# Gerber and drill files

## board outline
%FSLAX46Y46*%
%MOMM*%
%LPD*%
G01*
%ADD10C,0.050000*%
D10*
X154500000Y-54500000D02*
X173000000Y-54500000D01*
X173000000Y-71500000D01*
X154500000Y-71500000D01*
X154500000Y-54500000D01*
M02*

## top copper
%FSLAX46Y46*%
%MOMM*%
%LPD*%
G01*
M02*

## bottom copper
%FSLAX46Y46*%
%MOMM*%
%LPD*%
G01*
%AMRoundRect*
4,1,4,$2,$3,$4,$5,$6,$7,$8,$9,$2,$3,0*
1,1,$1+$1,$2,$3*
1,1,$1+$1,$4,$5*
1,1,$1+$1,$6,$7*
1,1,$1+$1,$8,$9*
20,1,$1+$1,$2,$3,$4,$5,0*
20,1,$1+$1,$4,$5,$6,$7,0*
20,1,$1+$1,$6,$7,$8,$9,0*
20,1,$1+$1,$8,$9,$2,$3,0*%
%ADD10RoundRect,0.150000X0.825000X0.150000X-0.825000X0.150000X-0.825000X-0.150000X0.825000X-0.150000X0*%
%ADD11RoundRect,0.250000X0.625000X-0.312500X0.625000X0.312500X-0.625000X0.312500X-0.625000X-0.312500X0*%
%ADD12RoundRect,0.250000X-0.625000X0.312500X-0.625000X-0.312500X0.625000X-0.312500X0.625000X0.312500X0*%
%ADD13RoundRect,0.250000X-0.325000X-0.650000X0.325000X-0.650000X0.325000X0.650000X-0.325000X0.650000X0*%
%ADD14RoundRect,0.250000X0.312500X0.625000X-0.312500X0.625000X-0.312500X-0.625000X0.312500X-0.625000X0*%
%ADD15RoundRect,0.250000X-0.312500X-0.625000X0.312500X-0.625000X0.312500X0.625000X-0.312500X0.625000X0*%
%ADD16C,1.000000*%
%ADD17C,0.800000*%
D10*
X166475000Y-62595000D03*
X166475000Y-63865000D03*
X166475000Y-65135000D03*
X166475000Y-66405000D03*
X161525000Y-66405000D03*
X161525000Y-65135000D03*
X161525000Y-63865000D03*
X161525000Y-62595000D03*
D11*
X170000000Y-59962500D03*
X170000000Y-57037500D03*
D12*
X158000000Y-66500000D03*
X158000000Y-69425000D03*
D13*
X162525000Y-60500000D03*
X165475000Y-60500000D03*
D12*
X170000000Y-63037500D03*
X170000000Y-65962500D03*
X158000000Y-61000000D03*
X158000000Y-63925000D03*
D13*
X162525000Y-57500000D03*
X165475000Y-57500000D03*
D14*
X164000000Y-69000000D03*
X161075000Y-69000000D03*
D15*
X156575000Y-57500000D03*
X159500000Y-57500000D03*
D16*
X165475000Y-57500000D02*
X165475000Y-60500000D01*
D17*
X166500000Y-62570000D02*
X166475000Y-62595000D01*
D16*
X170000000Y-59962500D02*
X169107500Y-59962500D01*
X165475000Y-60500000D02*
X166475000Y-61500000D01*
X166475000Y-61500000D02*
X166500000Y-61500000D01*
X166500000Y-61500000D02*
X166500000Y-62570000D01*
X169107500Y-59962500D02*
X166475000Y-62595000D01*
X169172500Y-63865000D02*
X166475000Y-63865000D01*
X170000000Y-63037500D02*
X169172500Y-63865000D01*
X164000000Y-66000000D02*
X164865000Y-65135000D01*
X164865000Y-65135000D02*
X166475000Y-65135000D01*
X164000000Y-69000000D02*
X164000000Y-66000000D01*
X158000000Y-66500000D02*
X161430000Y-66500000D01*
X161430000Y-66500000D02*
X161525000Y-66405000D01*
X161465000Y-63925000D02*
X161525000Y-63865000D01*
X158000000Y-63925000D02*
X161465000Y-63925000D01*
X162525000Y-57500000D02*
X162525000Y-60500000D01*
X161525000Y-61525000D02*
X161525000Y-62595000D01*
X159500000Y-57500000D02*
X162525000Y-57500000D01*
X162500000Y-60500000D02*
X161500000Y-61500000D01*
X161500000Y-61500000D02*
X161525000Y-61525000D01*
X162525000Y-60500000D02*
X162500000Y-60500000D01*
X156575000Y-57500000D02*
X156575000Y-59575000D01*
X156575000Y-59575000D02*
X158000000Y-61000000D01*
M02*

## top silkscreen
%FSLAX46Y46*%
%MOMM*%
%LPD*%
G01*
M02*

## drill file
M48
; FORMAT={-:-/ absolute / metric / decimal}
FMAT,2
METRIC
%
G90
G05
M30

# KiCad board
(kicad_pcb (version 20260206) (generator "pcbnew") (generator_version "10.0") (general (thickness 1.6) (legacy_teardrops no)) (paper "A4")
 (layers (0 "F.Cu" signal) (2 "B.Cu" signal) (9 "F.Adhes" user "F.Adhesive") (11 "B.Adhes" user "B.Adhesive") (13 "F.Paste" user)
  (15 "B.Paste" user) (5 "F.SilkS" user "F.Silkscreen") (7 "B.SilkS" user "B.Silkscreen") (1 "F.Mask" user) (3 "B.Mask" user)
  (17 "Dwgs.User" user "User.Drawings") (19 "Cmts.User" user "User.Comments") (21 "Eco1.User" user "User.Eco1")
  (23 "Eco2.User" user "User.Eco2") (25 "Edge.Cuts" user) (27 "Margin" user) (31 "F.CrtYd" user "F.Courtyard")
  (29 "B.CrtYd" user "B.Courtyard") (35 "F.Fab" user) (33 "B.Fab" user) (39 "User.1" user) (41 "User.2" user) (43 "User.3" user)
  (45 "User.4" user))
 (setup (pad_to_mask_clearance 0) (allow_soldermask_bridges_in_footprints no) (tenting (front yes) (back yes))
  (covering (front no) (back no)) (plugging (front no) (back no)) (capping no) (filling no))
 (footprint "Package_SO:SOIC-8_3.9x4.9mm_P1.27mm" (layer "B.Cu") (at 164 64.5 180)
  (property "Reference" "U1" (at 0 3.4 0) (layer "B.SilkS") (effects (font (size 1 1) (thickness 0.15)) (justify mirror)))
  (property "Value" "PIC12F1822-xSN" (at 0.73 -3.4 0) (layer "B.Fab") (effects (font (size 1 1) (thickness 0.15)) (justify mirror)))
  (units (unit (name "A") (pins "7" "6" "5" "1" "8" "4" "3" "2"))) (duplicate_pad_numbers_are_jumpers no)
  (pad "1" smd roundrect (at -2.475 1.905 180) (size 1.95 0.6) (layers "B.Cu" "B.Mask" "B.Paste") (roundrect_rratio 0.25)
   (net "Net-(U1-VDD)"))
  (pad "2" smd roundrect (at -2.475 0.635 180) (size 1.95 0.6) (layers "B.Cu" "B.Mask" "B.Paste") (roundrect_rratio 0.25)
   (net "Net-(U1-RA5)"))
  (pad "3" smd roundrect (at -2.475 -0.635 180) (size 1.95 0.6) (layers "B.Cu" "B.Mask" "B.Paste") (roundrect_rratio 0.25)
   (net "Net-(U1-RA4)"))
  (pad "4" smd roundrect (at -2.475 -1.905 180) (size 1.95 0.6) (layers "B.Cu" "B.Mask" "B.Paste") (roundrect_rratio 0.25)
   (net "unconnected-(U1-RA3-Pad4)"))
  (pad "5" smd roundrect (at 2.475 -1.905 180) (size 1.95 0.6) (layers "B.Cu" "B.Mask" "B.Paste") (roundrect_rratio 0.25)
   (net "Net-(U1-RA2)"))
  (pad "6" smd roundrect (at 2.475 -0.635 180) (size 1.95 0.6) (layers "B.Cu" "B.Mask" "B.Paste") (roundrect_rratio 0.25)
   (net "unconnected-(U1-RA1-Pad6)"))
  (pad "7" smd roundrect (at 2.475 0.635 180) (size 1.95 0.6) (layers "B.Cu" "B.Mask" "B.Paste") (roundrect_rratio 0.25)
   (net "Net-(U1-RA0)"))
  (pad "8" smd roundrect (at 2.475 1.905 180) (size 1.95 0.6) (layers "B.Cu" "B.Mask" "B.Paste") (roundrect_rratio 0.25) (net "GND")))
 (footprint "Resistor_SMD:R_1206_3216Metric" (layer "B.Cu") (at 170 58.5 90)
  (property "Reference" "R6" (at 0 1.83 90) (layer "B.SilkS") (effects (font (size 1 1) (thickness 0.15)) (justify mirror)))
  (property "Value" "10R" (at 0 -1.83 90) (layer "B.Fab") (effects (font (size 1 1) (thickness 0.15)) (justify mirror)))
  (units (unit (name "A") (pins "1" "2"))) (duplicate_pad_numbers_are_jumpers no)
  (pad "1" smd roundrect (at -1.4625 0 90) (size 1.125 1.75) (layers "B.Cu" "B.Mask" "B.Paste") (roundrect_rratio 0.222222)
   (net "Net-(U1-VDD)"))
  (pad "2" smd roundrect (at 1.4625 0 90) (size 1.125 1.75) (layers "B.Cu" "B.Mask" "B.Paste") (roundrect_rratio 0.222222) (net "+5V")))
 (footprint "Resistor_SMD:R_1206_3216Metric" (layer "B.Cu") (at 158 67.9625 -90)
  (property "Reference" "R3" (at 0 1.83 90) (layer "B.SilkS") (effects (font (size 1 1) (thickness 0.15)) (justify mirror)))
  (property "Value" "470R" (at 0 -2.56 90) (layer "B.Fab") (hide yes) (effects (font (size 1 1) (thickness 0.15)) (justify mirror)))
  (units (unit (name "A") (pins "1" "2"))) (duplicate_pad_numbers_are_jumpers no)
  (pad "1" smd roundrect (at -1.4625 0 270) (size 1.125 1.75) (layers "B.Cu" "B.Mask" "B.Paste") (roundrect_rratio 0.222222)
   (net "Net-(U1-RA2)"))
  (pad "2" smd roundrect (at 1.4625 0 270) (size 1.125 1.75) (layers "B.Cu" "B.Mask" "B.Paste") (roundrect_rratio 0.222222)
   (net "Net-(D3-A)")))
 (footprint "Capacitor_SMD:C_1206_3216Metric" (layer "B.Cu") (at 164 60.5)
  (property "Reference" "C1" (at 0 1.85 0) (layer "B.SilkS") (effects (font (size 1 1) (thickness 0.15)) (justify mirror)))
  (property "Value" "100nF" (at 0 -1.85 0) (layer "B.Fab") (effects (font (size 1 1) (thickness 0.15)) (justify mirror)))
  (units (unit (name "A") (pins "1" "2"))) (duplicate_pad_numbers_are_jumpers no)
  (pad "1" smd roundrect (at -1.475 0) (size 1.15 1.8) (layers "B.Cu" "B.Mask" "B.Paste") (roundrect_rratio 0.217391) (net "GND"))
  (pad "2" smd roundrect (at 1.475 0) (size 1.15 1.8) (layers "B.Cu" "B.Mask" "B.Paste") (roundrect_rratio 0.217391) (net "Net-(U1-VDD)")))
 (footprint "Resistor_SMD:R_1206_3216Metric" (layer "B.Cu") (at 170 64.5 -90)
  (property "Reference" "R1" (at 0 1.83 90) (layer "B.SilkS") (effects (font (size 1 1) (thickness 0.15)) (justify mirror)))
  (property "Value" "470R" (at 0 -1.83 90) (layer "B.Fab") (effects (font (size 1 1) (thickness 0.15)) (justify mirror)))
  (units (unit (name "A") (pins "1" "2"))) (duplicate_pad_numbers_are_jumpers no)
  (pad "1" smd roundrect (at -1.4625 0 270) (size 1.125 1.75) (layers "B.Cu" "B.Mask" "B.Paste") (roundrect_rratio 0.222222)
   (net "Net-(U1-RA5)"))
  (pad "2" smd roundrect (at 1.4625 0 270) (size 1.125 1.75) (layers "B.Cu" "B.Mask" "B.Paste") (roundrect_rratio 0.222222)
   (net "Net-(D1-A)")))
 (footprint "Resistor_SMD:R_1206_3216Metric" (layer "B.Cu") (at 158 62.4625 -90)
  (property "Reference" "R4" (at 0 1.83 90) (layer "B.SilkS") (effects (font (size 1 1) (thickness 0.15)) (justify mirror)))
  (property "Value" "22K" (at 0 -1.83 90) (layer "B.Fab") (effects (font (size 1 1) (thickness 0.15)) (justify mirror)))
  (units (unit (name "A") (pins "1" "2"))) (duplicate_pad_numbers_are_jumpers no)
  (pad "1" smd roundrect (at -1.4625 0 270) (size 1.125 1.75) (layers "B.Cu" "B.Mask" "B.Paste") (roundrect_rratio 0.222222)
   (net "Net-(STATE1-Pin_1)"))
  (pad "2" smd roundrect (at 1.4625 0 270) (size 1.125 1.75) (layers "B.Cu" "B.Mask" "B.Paste") (roundrect_rratio 0.222222)
   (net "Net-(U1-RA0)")))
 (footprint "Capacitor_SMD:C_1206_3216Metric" (layer "B.Cu") (at 164 57.5)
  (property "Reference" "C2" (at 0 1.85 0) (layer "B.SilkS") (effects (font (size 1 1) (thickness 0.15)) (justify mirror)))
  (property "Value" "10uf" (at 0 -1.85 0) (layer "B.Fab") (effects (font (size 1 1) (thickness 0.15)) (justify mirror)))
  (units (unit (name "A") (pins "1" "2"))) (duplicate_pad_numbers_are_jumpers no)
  (pad "1" smd roundrect (at -1.475 0) (size 1.15 1.8) (layers "B.Cu" "B.Mask" "B.Paste") (roundrect_rratio 0.217391) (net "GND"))
  (pad "2" smd roundrect (at 1.475 0) (size 1.15 1.8) (layers "B.Cu" "B.Mask" "B.Paste") (roundrect_rratio 0.217391) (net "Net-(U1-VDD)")))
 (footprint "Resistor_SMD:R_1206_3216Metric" (layer "B.Cu") (at 162.5375 69 180)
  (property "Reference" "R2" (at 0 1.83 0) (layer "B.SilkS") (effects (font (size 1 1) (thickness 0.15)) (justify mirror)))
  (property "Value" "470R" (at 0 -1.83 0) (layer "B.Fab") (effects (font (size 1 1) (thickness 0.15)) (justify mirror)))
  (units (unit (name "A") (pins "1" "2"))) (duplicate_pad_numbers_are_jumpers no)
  (pad "1" smd roundrect (at -1.4625 0 180) (size 1.125 1.75) (layers "B.Cu" "B.Mask" "B.Paste") (roundrect_rratio 0.222222)
   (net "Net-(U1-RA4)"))
  (pad "2" smd roundrect (at 1.4625 0 180) (size 1.125 1.75) (layers "B.Cu" "B.Mask" "B.Paste") (roundrect_rratio 0.222222)
   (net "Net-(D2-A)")))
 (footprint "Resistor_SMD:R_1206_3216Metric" (layer "B.Cu") (at 158.0375 57.5)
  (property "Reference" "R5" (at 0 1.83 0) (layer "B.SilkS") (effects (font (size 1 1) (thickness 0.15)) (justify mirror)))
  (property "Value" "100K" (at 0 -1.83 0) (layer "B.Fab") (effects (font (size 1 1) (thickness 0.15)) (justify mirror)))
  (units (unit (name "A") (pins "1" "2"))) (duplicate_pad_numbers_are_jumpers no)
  (pad "1" smd roundrect (at -1.4625 0) (size 1.125 1.75) (layers "B.Cu" "B.Mask" "B.Paste") (roundrect_rratio 0.222222)
   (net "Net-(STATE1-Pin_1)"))
  (pad "2" smd roundrect (at 1.4625 0) (size 1.125 1.75) (layers "B.Cu" "B.Mask" "B.Paste") (roundrect_rratio 0.222222) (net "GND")))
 (gr_rect (start 154.5 54.5) (end 173 71.5) (stroke (width 0.05) (type default)) (fill no) (layer "Edge.Cuts"))
 (segment (start 165.475 57.5) (end 165.475 60.5) (width 1) (layer "B.Cu") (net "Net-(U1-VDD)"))
 (segment (start 166.5 62.57) (end 166.475 62.595) (width 0.8) (layer "B.Cu") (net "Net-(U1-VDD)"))
 (segment (start 170 59.9625) (end 169.1075 59.9625) (width 1) (layer "B.Cu") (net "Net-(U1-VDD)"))
 (segment (start 165.475 60.5) (end 166.475 61.5) (width 1) (layer "B.Cu") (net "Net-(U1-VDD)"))
 (segment (start 166.475 61.5) (end 166.5 61.5) (width 1) (layer "B.Cu") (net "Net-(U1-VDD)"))
 (segment (start 166.5 61.5) (end 166.5 62.57) (width 1) (layer "B.Cu") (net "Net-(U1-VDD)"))
 (segment (start 169.1075 59.9625) (end 166.475 62.595) (width 1) (layer "B.Cu") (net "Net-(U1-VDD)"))
 (segment (start 169.1725 63.865) (end 166.475 63.865) (width 1) (layer "B.Cu") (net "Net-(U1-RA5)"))
 (segment (start 170 63.0375) (end 169.1725 63.865) (width 1) (layer "B.Cu") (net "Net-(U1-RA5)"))
 (segment (start 164 66) (end 164.865 65.135) (width 1) (layer "B.Cu") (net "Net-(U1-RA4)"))
 (segment (start 164.865 65.135) (end 166.475 65.135) (width 1) (layer "B.Cu") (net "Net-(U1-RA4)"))
 (segment (start 164 69) (end 164 66) (width 1) (layer "B.Cu") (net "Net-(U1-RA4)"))
 (segment (start 158 66.5) (end 161.43 66.5) (width 1) (layer "B.Cu") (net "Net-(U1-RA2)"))
 (segment (start 161.43 66.5) (end 161.525 66.405) (width 1) (layer "B.Cu") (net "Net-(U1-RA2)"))
 (segment (start 161.465 63.925) (end 161.525 63.865) (width 1) (layer "B.Cu") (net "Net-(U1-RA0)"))
 (segment (start 158 63.925) (end 161.465 63.925) (width 1) (layer "B.Cu") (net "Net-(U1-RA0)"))
 (segment (start 162.525 57.5) (end 162.525 60.5) (width 1) (layer "B.Cu") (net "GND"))
 (segment (start 161.525 61.525) (end 161.525 62.595) (width 1) (layer "B.Cu") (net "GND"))
 (segment (start 159.5 57.5) (end 162.525 57.5) (width 1) (layer "B.Cu") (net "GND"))
 (segment (start 162.5 60.5) (end 161.5 61.5) (width 1) (layer "B.Cu") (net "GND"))
 (segment (start 161.5 61.5) (end 161.525 61.525) (width 1) (layer "B.Cu") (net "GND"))
 (segment (start 162.525 60.5) (end 162.5 60.5) (width 1) (layer "B.Cu") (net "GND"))
 (segment (start 156.575 57.5) (end 156.575 59.575) (width 1) (layer "B.Cu") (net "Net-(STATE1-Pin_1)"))
 (segment (start 156.575 59.575) (end 158 61) (width 1) (layer "B.Cu") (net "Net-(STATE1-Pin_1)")))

